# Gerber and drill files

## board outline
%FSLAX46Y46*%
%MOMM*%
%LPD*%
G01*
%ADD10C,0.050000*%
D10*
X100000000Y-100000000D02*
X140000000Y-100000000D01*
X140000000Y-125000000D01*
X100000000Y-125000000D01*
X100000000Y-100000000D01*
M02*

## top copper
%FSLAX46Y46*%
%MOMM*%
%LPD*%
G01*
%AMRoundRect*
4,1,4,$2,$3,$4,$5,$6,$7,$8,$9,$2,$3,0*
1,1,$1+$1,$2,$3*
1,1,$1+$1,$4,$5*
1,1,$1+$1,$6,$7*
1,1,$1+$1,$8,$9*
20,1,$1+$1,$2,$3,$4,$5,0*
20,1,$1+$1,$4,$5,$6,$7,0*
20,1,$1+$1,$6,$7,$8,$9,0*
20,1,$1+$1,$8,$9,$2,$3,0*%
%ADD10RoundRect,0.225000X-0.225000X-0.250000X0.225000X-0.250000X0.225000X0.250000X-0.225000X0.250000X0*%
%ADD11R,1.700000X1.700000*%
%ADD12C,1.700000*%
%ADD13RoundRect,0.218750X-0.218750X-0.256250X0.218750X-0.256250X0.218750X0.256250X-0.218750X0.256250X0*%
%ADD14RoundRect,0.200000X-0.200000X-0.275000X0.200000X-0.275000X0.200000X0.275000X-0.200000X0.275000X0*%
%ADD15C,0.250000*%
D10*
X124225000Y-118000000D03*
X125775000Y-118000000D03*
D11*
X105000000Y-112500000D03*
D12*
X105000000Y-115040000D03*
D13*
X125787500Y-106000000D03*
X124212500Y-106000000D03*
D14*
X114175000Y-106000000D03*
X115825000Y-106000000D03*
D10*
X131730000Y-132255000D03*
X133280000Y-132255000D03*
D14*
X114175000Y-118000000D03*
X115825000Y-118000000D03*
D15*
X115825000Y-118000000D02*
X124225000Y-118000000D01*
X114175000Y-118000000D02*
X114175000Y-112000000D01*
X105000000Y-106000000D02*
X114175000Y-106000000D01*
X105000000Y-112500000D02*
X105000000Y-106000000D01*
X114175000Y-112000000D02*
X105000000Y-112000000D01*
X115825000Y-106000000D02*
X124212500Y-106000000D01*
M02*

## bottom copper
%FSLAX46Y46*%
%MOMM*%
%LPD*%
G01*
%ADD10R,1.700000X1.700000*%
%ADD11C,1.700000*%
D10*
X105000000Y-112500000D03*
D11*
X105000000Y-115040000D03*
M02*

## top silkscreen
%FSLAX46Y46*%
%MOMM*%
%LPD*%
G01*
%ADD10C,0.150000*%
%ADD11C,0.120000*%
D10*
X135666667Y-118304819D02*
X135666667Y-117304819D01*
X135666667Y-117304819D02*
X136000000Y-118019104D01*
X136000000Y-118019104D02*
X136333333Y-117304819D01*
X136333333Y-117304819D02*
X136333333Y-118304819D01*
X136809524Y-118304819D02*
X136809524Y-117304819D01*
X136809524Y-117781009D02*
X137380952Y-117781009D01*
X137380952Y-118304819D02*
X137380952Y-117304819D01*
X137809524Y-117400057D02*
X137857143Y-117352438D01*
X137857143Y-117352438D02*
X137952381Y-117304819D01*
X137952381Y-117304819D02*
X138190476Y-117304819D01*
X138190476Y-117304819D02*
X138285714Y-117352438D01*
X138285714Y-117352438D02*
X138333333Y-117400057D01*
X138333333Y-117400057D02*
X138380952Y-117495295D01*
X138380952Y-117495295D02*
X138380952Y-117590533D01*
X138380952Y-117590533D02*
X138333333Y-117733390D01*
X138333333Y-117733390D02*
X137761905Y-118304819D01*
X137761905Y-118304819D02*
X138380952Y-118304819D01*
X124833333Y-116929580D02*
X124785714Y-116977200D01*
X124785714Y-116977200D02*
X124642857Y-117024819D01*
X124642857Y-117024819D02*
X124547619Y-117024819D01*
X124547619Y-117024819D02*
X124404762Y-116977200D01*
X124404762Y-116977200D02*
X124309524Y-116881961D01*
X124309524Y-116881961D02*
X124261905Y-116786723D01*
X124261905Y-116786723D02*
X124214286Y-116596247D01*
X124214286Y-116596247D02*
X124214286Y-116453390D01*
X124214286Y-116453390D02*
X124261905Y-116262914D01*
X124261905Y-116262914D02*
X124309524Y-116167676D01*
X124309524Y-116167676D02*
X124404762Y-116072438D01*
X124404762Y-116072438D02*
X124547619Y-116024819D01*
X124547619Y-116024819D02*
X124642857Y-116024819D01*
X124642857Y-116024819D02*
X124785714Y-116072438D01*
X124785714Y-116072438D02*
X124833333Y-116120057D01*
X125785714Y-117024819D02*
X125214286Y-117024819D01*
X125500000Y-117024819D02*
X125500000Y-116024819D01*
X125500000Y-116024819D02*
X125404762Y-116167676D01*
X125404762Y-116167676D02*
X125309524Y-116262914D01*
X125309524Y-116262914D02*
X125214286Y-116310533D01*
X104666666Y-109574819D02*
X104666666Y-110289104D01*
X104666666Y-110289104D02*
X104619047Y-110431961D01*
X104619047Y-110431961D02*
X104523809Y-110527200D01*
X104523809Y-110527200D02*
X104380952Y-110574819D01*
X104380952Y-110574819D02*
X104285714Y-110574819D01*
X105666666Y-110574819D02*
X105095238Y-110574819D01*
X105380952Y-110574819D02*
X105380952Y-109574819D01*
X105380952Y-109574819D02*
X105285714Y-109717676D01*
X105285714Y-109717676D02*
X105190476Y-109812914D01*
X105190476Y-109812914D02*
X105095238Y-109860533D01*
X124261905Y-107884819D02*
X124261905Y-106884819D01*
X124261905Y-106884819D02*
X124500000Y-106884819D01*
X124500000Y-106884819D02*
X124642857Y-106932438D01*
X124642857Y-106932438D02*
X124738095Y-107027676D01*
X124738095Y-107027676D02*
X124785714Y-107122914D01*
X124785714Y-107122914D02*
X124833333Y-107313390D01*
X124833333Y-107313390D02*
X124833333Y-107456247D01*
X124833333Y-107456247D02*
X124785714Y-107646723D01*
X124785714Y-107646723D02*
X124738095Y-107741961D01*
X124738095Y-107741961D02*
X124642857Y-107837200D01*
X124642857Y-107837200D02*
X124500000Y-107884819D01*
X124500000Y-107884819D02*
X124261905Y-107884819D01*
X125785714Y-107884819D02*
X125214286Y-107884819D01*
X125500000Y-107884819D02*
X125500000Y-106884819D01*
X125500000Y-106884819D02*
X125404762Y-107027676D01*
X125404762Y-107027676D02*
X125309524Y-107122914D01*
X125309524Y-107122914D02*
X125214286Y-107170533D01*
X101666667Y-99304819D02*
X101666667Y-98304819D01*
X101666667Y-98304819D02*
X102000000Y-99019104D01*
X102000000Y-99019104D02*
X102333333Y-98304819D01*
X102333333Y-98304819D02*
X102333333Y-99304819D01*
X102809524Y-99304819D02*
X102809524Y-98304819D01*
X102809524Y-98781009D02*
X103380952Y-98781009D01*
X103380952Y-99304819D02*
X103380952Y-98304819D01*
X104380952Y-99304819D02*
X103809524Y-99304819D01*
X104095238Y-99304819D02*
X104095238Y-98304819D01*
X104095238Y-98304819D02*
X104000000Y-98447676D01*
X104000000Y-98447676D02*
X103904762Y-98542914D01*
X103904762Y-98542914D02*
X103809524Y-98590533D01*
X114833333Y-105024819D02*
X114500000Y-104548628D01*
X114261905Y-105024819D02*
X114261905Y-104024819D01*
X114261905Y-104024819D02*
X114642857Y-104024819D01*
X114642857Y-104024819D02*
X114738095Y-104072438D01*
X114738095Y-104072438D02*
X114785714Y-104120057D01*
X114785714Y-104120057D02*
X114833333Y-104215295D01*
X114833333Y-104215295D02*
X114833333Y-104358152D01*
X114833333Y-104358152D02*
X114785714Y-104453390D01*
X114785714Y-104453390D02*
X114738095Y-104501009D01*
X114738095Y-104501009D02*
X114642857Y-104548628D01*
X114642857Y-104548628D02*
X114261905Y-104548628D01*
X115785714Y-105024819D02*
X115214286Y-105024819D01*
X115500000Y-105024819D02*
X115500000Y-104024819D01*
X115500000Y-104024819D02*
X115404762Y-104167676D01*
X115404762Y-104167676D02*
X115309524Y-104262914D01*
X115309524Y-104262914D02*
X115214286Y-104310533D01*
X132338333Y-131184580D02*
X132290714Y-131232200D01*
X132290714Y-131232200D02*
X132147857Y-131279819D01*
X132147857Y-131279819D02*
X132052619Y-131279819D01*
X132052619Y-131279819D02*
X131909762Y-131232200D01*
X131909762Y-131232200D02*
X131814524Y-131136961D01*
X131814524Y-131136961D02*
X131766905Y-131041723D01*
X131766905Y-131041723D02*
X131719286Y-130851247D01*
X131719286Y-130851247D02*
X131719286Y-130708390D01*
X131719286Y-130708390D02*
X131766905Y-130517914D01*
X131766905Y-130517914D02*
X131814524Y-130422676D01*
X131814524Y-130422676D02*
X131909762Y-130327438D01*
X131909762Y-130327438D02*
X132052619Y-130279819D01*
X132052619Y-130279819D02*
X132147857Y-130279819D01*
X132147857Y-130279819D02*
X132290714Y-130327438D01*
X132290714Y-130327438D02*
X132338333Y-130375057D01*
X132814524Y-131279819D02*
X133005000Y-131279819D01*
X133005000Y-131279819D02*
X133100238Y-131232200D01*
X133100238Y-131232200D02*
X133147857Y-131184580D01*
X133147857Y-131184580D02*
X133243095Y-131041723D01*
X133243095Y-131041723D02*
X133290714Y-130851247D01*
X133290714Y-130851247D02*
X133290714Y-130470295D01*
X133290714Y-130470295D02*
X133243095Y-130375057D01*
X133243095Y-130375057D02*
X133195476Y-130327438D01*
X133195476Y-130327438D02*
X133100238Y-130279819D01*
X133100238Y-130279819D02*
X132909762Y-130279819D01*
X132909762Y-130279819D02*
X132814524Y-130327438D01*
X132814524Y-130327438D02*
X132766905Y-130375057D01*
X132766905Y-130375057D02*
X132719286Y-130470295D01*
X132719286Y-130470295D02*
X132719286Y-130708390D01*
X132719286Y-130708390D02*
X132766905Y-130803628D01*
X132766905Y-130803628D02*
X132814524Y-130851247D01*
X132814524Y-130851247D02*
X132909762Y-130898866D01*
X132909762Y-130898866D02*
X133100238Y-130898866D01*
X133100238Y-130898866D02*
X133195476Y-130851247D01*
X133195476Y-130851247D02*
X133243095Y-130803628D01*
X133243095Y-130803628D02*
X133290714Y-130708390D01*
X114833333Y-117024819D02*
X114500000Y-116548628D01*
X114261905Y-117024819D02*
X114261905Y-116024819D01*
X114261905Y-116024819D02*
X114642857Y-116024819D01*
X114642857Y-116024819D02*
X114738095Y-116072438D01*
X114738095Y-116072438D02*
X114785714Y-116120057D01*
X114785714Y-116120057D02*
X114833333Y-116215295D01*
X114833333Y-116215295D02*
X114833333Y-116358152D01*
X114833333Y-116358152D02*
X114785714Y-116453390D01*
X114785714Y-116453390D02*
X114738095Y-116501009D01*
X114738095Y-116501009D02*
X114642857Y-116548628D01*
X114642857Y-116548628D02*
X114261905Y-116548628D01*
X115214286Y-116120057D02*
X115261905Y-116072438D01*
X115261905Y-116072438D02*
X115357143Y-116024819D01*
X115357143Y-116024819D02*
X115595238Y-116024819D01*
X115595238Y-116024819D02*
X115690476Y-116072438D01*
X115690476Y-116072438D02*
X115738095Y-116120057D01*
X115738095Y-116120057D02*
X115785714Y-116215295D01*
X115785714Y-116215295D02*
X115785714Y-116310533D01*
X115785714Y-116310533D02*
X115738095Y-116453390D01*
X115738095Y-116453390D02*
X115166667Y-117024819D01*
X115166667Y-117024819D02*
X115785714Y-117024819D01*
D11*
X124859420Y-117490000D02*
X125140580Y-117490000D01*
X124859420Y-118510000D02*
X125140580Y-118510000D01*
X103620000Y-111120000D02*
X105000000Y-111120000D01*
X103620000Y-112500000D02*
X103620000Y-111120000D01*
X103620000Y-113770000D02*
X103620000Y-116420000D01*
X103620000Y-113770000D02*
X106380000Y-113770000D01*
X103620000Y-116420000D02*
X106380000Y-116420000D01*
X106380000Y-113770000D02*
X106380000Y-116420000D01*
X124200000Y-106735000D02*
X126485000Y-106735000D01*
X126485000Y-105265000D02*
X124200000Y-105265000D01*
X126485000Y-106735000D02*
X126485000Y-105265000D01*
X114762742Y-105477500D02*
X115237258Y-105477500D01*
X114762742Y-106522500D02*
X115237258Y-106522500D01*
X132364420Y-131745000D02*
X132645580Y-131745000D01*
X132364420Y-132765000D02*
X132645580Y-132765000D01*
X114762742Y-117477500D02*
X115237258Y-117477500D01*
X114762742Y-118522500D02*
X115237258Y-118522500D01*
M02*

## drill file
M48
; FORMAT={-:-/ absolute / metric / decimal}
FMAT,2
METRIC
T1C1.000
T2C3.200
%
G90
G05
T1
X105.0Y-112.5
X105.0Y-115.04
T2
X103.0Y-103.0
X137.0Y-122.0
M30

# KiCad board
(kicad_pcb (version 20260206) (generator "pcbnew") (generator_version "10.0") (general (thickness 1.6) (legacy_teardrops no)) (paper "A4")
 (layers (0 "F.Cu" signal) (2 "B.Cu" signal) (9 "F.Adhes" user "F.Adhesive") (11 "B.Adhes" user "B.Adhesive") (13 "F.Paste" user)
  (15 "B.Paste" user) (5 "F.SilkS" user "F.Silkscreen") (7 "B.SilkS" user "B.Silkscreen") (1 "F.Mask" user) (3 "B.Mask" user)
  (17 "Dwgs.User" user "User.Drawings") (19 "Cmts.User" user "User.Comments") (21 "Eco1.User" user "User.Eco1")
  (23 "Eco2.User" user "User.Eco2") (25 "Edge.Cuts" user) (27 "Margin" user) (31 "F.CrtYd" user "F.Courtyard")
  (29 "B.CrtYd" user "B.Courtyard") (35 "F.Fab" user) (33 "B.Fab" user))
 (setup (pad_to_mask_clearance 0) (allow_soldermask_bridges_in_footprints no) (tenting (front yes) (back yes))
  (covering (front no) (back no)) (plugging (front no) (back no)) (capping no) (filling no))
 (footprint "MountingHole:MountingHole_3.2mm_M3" (layer "F.Cu") (at 137 122)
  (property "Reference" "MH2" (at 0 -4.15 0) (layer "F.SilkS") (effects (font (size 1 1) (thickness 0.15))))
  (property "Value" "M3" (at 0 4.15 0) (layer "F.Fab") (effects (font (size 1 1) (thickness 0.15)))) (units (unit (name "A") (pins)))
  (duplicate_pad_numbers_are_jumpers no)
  (pad "" np_thru_hole circle (at 0 0) (size 3.2 3.2) (drill 3.2) (layers "*.Cu" "*.Mask")))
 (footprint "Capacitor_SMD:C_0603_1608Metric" (layer "F.Cu") (at 125 118)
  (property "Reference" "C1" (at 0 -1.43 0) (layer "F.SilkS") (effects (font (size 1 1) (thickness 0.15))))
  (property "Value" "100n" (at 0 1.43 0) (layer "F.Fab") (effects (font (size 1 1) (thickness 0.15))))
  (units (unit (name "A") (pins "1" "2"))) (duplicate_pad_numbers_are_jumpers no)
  (fp_line (start -0.14058 -0.51) (end 0.14058 -0.51) (stroke (width 0.12) (type solid)) (layer "F.SilkS"))
  (fp_line (start -0.14058 0.51) (end 0.14058 0.51) (stroke (width 0.12) (type solid)) (layer "F.SilkS"))
  (pad "1" smd roundrect (at -0.775 0) (size 0.9 0.95) (layers "F.Cu" "F.Mask" "F.Paste") (roundrect_rratio 0.25) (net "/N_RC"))
  (pad "2" smd roundrect (at 0.775 0) (size 0.9 0.95) (layers "F.Cu" "F.Mask" "F.Paste") (roundrect_rratio 0.25) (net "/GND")))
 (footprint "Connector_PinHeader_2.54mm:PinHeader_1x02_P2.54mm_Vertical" (layer "F.Cu") (at 105 112.5)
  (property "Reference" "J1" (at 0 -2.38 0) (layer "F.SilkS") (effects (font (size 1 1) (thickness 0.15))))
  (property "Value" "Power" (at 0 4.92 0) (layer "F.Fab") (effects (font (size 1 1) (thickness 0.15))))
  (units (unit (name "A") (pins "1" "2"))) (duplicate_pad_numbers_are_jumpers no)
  (fp_line (start -1.38 -1.38) (end 0 -1.38) (stroke (width 0.12) (type solid)) (layer "F.SilkS"))
  (fp_line (start -1.38 0) (end -1.38 -1.38) (stroke (width 0.12) (type solid)) (layer "F.SilkS"))
  (fp_line (start -1.38 1.27) (end -1.38 3.92) (stroke (width 0.12) (type solid)) (layer "F.SilkS"))
  (fp_line (start -1.38 1.27) (end 1.38 1.27) (stroke (width 0.12) (type solid)) (layer "F.SilkS"))
  (fp_line (start -1.38 3.92) (end 1.38 3.92) (stroke (width 0.12) (type solid)) (layer "F.SilkS"))
  (fp_line (start 1.38 1.27) (end 1.38 3.92) (stroke (width 0.12) (type solid)) (layer "F.SilkS"))
  (pad "1" thru_hole rect (at 0 0) (size 1.7 1.7) (drill 1) (layers "*.Cu" "*.Mask") (remove_unused_layers no) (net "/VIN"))
  (pad "2" thru_hole circle (at 0 2.54) (size 1.7 1.7) (drill 1) (layers "*.Cu" "*.Mask") (remove_unused_layers no) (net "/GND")))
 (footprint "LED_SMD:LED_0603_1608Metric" (layer "F.Cu") (at 125 106 180)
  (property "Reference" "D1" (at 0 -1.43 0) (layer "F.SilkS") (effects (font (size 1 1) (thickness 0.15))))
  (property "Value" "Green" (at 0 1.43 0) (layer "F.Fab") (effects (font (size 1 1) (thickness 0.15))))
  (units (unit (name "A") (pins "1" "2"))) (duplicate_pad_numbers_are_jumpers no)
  (fp_line (start 0.8 -0.735) (end -1.485 -0.735) (stroke (width 0.12) (type solid)) (layer "F.SilkS"))
  (fp_line (start -1.485 0.735) (end 0.8 0.735) (stroke (width 0.12) (type solid)) (layer "F.SilkS"))
  (fp_line (start -1.485 -0.735) (end -1.485 0.735) (stroke (width 0.12) (type solid)) (layer "F.SilkS"))
  (pad "1" smd roundrect (at -0.7875 0) (size 0.875 0.95) (layers "F.Cu" "F.Mask" "F.Paste") (roundrect_rratio 0.25) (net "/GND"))
  (pad "2" smd roundrect (at 0.7875 0) (size 0.875 0.95) (layers "F.Cu" "F.Mask" "F.Paste") (roundrect_rratio 0.25) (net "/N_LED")))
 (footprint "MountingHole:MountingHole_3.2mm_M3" (layer "F.Cu") (at 103 103)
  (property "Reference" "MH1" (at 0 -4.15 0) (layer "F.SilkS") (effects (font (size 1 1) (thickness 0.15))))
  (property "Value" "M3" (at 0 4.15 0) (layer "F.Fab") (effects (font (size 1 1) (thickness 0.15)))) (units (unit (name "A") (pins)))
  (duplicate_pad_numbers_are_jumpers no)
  (pad "" np_thru_hole circle (at 0 0) (size 3.2 3.2) (drill 3.2) (layers "*.Cu" "*.Mask")))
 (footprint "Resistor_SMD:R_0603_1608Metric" (layer "F.Cu") (at 115 106)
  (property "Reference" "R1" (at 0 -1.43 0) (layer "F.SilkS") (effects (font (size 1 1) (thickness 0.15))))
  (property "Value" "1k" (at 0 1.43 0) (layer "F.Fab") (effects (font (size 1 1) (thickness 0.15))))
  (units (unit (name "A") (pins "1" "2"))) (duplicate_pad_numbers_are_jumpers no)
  (fp_line (start -0.237258 -0.5225) (end 0.237258 -0.5225) (stroke (width 0.12) (type solid)) (layer "F.SilkS"))
  (fp_line (start -0.237258 0.5225) (end 0.237258 0.5225) (stroke (width 0.12) (type solid)) (layer "F.SilkS"))
  (pad "1" smd roundrect (at -0.825 0) (size 0.8 0.95) (layers "F.Cu" "F.Mask" "F.Paste") (roundrect_rratio 0.25) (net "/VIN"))
  (pad "2" smd roundrect (at 0.825 0) (size 0.8 0.95) (layers "F.Cu" "F.Mask" "F.Paste") (roundrect_rratio 0.25) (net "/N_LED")))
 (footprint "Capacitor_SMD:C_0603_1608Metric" (layer "F.Cu") (at 132.505 132.255)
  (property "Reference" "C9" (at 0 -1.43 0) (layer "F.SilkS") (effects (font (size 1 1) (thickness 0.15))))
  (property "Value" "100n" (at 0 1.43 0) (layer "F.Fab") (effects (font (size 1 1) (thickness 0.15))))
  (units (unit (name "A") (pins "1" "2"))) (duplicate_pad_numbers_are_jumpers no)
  (fp_line (start -0.14058 -0.51) (end 0.14058 -0.51) (stroke (width 0.12) (type solid)) (layer "F.SilkS"))
  (fp_line (start -0.14058 0.51) (end 0.14058 0.51) (stroke (width 0.12) (type solid)) (layer "F.SilkS"))
  (pad "1" smd roundrect (at -0.775 0) (size 0.9 0.95) (layers "F.Cu" "F.Mask" "F.Paste") (roundrect_rratio 0.25) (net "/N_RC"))
  (pad "2" smd roundrect (at 0.775 0) (size 0.9 0.95) (layers "F.Cu" "F.Mask" "F.Paste") (roundrect_rratio 0.25) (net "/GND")))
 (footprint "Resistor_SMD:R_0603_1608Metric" (layer "F.Cu") (at 115 118)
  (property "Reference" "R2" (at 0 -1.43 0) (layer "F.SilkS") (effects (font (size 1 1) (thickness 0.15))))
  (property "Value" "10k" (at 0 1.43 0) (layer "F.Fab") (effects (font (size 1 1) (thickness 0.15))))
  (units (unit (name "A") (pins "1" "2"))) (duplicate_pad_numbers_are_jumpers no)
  (fp_line (start -0.237258 -0.5225) (end 0.237258 -0.5225) (stroke (width 0.12) (type solid)) (layer "F.SilkS"))
  (fp_line (start -0.237258 0.5225) (end 0.237258 0.5225) (stroke (width 0.12) (type solid)) (layer "F.SilkS"))
  (pad "1" smd roundrect (at -0.825 0) (size 0.8 0.95) (layers "F.Cu" "F.Mask" "F.Paste") (roundrect_rratio 0.25) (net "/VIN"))
  (pad "2" smd roundrect (at 0.825 0) (size 0.8 0.95) (layers "F.Cu" "F.Mask" "F.Paste") (roundrect_rratio 0.25) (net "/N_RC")))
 (gr_rect (start 100 100) (end 140 125) (stroke (width 0.05) (type default)) (fill no) (layer "Edge.Cuts"))
 (segment (start 115.825 118) (end 124.225 118) (width 0.25) (layer "F.Cu") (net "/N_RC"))
 (segment (start 114.175 118) (end 114.175 112) (width 0.25) (layer "F.Cu") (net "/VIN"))
 (segment (start 105 106) (end 114.175 106) (width 0.25) (layer "F.Cu") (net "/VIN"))
 (segment (start 105 112.5) (end 105 106) (width 0.25) (layer "F.Cu") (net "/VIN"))
 (segment (start 114.175 112) (end 105 112) (width 0.25) (layer "F.Cu") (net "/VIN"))
 (segment (start 115.825 106) (end 124.2125 106) (width 0.25) (layer "F.Cu") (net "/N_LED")))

